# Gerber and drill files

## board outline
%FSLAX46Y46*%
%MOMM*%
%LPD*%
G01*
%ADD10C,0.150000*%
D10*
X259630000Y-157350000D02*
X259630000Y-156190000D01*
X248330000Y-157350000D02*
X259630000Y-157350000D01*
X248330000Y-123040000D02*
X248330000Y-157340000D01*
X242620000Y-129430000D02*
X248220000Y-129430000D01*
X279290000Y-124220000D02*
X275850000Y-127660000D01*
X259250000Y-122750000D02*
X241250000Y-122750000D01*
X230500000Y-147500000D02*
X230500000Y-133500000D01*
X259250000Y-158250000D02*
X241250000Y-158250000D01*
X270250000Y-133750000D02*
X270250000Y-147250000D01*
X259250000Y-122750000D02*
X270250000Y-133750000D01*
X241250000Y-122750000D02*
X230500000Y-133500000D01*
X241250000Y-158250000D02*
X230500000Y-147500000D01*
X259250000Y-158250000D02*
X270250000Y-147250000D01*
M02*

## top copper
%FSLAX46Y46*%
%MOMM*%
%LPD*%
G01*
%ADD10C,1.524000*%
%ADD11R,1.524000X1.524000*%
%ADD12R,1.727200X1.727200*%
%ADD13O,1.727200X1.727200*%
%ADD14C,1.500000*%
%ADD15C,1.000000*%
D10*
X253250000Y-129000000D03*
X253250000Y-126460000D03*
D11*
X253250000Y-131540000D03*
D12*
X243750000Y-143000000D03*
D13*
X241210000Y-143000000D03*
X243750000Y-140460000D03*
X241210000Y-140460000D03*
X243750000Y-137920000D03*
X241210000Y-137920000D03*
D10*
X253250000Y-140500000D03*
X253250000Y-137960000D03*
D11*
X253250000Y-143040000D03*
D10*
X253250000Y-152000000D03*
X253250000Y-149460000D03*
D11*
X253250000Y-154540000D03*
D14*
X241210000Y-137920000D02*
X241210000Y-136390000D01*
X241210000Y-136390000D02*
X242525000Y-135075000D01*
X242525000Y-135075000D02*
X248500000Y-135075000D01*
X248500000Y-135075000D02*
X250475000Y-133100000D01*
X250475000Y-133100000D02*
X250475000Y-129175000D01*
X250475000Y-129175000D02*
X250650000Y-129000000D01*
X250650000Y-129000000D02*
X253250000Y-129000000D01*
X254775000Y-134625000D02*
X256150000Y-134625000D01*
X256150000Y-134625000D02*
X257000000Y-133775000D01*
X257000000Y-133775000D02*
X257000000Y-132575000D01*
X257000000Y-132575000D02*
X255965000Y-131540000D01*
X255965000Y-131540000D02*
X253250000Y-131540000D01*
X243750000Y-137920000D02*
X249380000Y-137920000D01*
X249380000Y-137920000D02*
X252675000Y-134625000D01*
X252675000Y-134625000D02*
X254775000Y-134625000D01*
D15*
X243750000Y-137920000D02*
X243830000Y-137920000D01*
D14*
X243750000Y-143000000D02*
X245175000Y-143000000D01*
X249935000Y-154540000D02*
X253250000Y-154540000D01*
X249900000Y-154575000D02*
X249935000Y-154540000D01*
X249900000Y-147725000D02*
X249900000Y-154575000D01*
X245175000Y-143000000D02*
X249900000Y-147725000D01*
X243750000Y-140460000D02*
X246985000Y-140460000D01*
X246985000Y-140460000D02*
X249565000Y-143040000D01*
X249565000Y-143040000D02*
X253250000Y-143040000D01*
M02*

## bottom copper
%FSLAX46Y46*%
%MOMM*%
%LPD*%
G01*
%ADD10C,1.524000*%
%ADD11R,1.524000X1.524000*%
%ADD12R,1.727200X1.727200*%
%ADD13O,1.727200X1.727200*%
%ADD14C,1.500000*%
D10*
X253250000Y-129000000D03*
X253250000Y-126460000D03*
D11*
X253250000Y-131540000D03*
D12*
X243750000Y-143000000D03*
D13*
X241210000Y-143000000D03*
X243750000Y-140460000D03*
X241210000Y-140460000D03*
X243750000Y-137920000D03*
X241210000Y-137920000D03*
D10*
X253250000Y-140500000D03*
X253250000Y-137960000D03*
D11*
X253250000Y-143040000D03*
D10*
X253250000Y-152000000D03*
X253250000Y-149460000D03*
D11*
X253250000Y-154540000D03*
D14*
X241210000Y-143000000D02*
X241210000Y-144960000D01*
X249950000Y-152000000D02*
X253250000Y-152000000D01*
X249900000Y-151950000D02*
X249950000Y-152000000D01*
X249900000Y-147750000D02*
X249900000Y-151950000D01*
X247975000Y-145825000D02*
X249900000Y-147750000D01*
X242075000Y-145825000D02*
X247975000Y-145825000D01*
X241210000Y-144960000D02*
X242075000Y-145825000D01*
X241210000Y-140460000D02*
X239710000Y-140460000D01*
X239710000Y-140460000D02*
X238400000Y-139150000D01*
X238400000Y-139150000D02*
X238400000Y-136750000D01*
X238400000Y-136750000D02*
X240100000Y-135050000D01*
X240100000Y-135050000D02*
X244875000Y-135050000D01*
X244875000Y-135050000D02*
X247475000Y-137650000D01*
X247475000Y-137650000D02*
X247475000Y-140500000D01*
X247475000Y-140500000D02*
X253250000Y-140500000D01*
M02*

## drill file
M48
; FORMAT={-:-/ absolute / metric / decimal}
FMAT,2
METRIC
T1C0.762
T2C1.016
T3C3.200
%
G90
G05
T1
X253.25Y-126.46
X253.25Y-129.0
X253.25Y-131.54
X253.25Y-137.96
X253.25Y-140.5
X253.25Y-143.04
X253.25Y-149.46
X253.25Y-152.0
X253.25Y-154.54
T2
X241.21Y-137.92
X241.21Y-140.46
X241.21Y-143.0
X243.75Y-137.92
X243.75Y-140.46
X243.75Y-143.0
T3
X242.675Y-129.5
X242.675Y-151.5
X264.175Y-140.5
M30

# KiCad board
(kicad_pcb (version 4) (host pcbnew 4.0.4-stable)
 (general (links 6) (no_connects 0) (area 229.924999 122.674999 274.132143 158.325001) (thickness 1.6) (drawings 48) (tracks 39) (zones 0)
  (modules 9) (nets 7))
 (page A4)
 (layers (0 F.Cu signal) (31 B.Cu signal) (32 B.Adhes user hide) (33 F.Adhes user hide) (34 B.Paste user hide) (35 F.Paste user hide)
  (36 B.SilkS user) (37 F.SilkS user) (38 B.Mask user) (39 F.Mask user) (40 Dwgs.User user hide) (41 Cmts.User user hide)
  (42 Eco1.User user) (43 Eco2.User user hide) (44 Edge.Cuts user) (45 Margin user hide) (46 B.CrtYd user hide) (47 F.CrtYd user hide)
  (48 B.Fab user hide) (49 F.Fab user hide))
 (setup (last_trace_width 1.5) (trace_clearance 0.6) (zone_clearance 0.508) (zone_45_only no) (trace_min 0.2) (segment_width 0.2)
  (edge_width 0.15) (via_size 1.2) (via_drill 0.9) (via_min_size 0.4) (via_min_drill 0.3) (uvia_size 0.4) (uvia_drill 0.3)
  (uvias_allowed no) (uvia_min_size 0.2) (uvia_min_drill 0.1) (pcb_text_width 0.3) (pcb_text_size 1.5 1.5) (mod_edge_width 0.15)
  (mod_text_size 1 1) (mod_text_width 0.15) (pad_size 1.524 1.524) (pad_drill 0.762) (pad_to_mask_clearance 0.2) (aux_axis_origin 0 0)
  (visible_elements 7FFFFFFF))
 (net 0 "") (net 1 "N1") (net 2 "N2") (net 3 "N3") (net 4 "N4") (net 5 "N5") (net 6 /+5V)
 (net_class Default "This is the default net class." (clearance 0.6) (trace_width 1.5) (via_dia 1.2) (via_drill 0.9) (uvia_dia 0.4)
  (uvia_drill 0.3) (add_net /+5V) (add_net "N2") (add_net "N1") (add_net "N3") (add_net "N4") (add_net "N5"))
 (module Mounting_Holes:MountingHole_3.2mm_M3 (layer F.Cu) (at 264.175 140.5)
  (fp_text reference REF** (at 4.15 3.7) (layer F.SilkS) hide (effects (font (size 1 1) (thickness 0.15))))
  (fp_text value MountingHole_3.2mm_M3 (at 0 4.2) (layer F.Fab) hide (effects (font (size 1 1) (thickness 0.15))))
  (pad 1 np_thru_hole circle (at 0 0) (size 3.2 3.2) (drill 3.2) (layers *.Cu *.Mask)))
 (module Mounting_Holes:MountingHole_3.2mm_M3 (layer F.Cu) (at 242.675 151.5)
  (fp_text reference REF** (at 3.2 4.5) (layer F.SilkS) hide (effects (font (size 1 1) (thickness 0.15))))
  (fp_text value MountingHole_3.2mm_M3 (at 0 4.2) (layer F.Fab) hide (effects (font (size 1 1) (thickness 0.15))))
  (pad 1 np_thru_hole circle (at 0 0) (size 3.2 3.2) (drill 3.2) (layers *.Cu *.Mask)))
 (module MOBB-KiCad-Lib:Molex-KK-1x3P (layer B.Cu) (at 253.25 129 270)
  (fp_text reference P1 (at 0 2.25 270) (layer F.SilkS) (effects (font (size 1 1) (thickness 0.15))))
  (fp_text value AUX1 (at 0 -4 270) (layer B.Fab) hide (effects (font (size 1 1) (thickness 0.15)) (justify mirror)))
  (pad 2 thru_hole circle (at 0 0 270) (size 1.524 1.524) (drill 0.762) (layers *.Cu *.Mask) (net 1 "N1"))
  (pad 3 thru_hole circle (at -2.54 0 270) (size 1.524 1.524) (drill 0.762) (layers *.Cu *.Mask))
  (pad 1 thru_hole rect (at 2.54 0 270) (size 1.524 1.524) (drill 0.762) (layers *.Cu *.Mask) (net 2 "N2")))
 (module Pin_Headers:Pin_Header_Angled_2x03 (layer F.Cu) (at 243.75 143 180)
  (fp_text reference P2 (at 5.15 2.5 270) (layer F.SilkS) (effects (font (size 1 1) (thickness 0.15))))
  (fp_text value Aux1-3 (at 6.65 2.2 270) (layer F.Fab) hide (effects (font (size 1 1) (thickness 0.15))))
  (pad 1 thru_hole rect (at 0 0 180) (size 1.7272 1.7272) (drill 1.016) (layers *.Cu *.Mask) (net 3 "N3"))
  (pad 2 thru_hole oval (at 2.54 0 180) (size 1.7272 1.7272) (drill 1.016) (layers *.Cu *.Mask) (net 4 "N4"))
  (pad 3 thru_hole oval (at 0 2.54 180) (size 1.7272 1.7272) (drill 1.016) (layers *.Cu *.Mask) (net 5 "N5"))
  (pad 4 thru_hole oval (at 2.54 2.54 180) (size 1.7272 1.7272) (drill 1.016) (layers *.Cu *.Mask) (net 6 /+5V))
  (pad 5 thru_hole oval (at 0 5.08 180) (size 1.7272 1.7272) (drill 1.016) (layers *.Cu *.Mask) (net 2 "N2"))
  (pad 6 thru_hole oval (at 2.54 5.08 180) (size 1.7272 1.7272) (drill 1.016) (layers *.Cu *.Mask) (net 1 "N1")))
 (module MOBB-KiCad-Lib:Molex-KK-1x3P (layer B.Cu) (at 253.25 140.5 270)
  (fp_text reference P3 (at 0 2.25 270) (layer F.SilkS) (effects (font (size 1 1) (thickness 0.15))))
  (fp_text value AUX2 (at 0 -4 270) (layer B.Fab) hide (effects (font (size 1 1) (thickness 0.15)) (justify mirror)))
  (pad 2 thru_hole circle (at 0 0 270) (size 1.524 1.524) (drill 0.762) (layers *.Cu *.Mask) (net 6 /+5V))
  (pad 3 thru_hole circle (at -2.54 0 270) (size 1.524 1.524) (drill 0.762) (layers *.Cu *.Mask))
  (pad 1 thru_hole rect (at 2.54 0 270) (size 1.524 1.524) (drill 0.762) (layers *.Cu *.Mask) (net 5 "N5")))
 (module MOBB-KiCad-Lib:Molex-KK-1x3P (layer B.Cu) (at 253.25 152 270)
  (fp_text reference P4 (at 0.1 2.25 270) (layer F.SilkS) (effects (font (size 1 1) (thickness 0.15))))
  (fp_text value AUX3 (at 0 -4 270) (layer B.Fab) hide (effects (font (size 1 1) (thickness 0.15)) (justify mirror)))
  (pad 2 thru_hole circle (at 0 0 270) (size 1.524 1.524) (drill 0.762) (layers *.Cu *.Mask) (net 4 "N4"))
  (pad 3 thru_hole circle (at -2.54 0 270) (size 1.524 1.524) (drill 0.762) (layers *.Cu *.Mask))
  (pad 1 thru_hole rect (at 2.54 0 270) (size 1.524 1.524) (drill 0.762) (layers *.Cu *.Mask) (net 3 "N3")))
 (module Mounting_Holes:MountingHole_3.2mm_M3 (layer F.Cu) (at 242.675 129.5)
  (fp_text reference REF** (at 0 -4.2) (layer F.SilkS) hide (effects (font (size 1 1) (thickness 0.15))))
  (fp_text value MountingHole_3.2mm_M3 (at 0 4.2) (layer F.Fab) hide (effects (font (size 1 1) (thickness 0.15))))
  (pad 1 np_thru_hole circle (at 0 0) (size 3.2 3.2) (drill 3.2) (layers *.Cu *.Mask)))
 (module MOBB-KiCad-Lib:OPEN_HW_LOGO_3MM (layer F.Cu) (at 237.1 130.5)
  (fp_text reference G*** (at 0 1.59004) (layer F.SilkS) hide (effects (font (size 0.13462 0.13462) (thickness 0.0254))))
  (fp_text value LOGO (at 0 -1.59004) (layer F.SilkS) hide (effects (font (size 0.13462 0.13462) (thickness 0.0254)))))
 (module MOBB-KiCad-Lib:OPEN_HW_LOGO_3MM (layer B.Cu) (at 237.1 130.5 180)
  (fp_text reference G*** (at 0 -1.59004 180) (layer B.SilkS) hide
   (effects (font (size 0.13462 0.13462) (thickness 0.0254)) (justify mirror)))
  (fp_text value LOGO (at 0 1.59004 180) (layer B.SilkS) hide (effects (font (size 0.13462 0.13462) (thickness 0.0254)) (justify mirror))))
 (gr_line (start 259.63 157.35) (end 259.63 156.19) (angle 90) (layer Edge.Cuts) (width 0.15))
 (gr_line (start 248.33 157.35) (end 259.63 157.35) (angle 90) (layer Edge.Cuts) (width 0.15))
 (gr_line (start 248.33 123.04) (end 248.33 157.34) (angle 90) (layer Edge.Cuts) (width 0.15))
 (gr_line (start 242.62 129.43) (end 248.22 129.43) (angle 90) (layer Edge.Cuts) (width 0.15))
 (gr_line (start 279.29 124.22) (end 275.85 127.66) (angle 90) (layer Edge.Cuts) (width 0.15))
 (gr_line (start 259.25 122.75) (end 241.25 122.75) (angle 90) (layer Edge.Cuts) (width 0.15))
 (gr_line (start 230.5 147.5) (end 230.5 133.5) (angle 90) (layer Edge.Cuts) (width 0.15))
 (gr_line (start 259.25 158.25) (end 241.25 158.25) (angle 90) (layer Edge.Cuts) (width 0.15))
 (gr_line (start 270.25 133.75) (end 270.25 147.25) (angle 90) (layer Edge.Cuts) (width 0.15))
 (gr_line (start 259.25 122.75) (end 270.25 133.75) (angle 90) (layer Edge.Cuts) (width 0.15))
 (gr_line (start 241.25 122.75) (end 230.5 133.5) (angle 90) (layer Edge.Cuts) (width 0.15))
 (gr_line (start 241.25 158.25) (end 230.5 147.5) (angle 90) (layer Edge.Cuts) (width 0.15))
 (gr_line (start 259.25 158.25) (end 270.25 147.25) (angle 90) (layer Edge.Cuts) (width 0.15))
 (segment (start 241.21 137.92) (end 241.21 136.39) (width 1.5) (layer F.Cu) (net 1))
 (segment (start 241.21 136.39) (end 242.525 135.075) (width 1.5) (layer F.Cu) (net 1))
 (segment (start 242.525 135.075) (end 248.5 135.075) (width 1.5) (layer F.Cu) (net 1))
 (segment (start 248.5 135.075) (end 250.475 133.1) (width 1.5) (layer F.Cu) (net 1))
 (segment (start 250.475 133.1) (end 250.475 129.175) (width 1.5) (layer F.Cu) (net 1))
 (segment (start 250.475 129.175) (end 250.65 129) (width 1.5) (layer F.Cu) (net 1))
 (segment (start 250.65 129) (end 253.25 129) (width 1.5) (layer F.Cu) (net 1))
 (segment (start 254.775 134.625) (end 256.15 134.625) (width 1.5) (layer F.Cu) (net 2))
 (segment (start 256.15 134.625) (end 257 133.775) (width 1.5) (layer F.Cu) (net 2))
 (segment (start 257 133.775) (end 257 132.575) (width 1.5) (layer F.Cu) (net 2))
 (segment (start 257 132.575) (end 255.965 131.54) (width 1.5) (layer F.Cu) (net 2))
 (segment (start 255.965 131.54) (end 253.25 131.54) (width 1.5) (layer F.Cu) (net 2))
 (segment (start 243.75 137.92) (end 249.38 137.92) (width 1.5) (layer F.Cu) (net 2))
 (segment (start 249.38 137.92) (end 252.675 134.625) (width 1.5) (layer F.Cu) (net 2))
 (segment (start 252.675 134.625) (end 254.775 134.625) (width 1.5) (layer F.Cu) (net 2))
 (segment (start 243.75 137.92) (end 243.83 137.92) (width 1) (layer F.Cu) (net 2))
 (segment (start 243.75 143) (end 245.175 143) (width 1.5) (layer F.Cu) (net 3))
 (segment (start 249.935 154.54) (end 253.25 154.54) (width 1.5) (layer F.Cu) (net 3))
 (segment (start 249.9 154.575) (end 249.935 154.54) (width 1.5) (layer F.Cu) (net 3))
 (segment (start 249.9 147.725) (end 249.9 154.575) (width 1.5) (layer F.Cu) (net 3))
 (segment (start 245.175 143) (end 249.9 147.725) (width 1.5) (layer F.Cu) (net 3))
 (segment (start 241.21 143) (end 241.21 144.96) (width 1.5) (layer B.Cu) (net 4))
 (segment (start 249.95 152) (end 253.25 152) (width 1.5) (layer B.Cu) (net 4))
 (segment (start 249.9 151.95) (end 249.95 152) (width 1.5) (layer B.Cu) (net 4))
 (segment (start 249.9 147.75) (end 249.9 151.95) (width 1.5) (layer B.Cu) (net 4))
 (segment (start 247.975 145.825) (end 249.9 147.75) (width 1.5) (layer B.Cu) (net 4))
 (segment (start 242.075 145.825) (end 247.975 145.825) (width 1.5) (layer B.Cu) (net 4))
 (segment (start 241.21 144.96) (end 242.075 145.825) (width 1.5) (layer B.Cu) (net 4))
 (segment (start 243.75 140.46) (end 246.985 140.46) (width 1.5) (layer F.Cu) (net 5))
 (segment (start 246.985 140.46) (end 249.565 143.04) (width 1.5) (layer F.Cu) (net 5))
 (segment (start 249.565 143.04) (end 253.25 143.04) (width 1.5) (layer F.Cu) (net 5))
 (segment (start 241.21 140.46) (end 239.71 140.46) (width 1.5) (layer B.Cu) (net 6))
 (segment (start 239.71 140.46) (end 238.4 139.15) (width 1.5) (layer B.Cu) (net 6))
 (segment (start 238.4 139.15) (end 238.4 136.75) (width 1.5) (layer B.Cu) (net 6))
 (segment (start 238.4 136.75) (end 240.1 135.05) (width 1.5) (layer B.Cu) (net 6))
 (segment (start 240.1 135.05) (end 244.875 135.05) (width 1.5) (layer B.Cu) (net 6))
 (segment (start 244.875 135.05) (end 247.475 137.65) (width 1.5) (layer B.Cu) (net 6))
 (segment (start 247.475 137.65) (end 247.475 140.5) (width 1.5) (layer B.Cu) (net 6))
 (segment (start 247.475 140.5) (end 253.25 140.5) (width 1.5) (layer B.Cu) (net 6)))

